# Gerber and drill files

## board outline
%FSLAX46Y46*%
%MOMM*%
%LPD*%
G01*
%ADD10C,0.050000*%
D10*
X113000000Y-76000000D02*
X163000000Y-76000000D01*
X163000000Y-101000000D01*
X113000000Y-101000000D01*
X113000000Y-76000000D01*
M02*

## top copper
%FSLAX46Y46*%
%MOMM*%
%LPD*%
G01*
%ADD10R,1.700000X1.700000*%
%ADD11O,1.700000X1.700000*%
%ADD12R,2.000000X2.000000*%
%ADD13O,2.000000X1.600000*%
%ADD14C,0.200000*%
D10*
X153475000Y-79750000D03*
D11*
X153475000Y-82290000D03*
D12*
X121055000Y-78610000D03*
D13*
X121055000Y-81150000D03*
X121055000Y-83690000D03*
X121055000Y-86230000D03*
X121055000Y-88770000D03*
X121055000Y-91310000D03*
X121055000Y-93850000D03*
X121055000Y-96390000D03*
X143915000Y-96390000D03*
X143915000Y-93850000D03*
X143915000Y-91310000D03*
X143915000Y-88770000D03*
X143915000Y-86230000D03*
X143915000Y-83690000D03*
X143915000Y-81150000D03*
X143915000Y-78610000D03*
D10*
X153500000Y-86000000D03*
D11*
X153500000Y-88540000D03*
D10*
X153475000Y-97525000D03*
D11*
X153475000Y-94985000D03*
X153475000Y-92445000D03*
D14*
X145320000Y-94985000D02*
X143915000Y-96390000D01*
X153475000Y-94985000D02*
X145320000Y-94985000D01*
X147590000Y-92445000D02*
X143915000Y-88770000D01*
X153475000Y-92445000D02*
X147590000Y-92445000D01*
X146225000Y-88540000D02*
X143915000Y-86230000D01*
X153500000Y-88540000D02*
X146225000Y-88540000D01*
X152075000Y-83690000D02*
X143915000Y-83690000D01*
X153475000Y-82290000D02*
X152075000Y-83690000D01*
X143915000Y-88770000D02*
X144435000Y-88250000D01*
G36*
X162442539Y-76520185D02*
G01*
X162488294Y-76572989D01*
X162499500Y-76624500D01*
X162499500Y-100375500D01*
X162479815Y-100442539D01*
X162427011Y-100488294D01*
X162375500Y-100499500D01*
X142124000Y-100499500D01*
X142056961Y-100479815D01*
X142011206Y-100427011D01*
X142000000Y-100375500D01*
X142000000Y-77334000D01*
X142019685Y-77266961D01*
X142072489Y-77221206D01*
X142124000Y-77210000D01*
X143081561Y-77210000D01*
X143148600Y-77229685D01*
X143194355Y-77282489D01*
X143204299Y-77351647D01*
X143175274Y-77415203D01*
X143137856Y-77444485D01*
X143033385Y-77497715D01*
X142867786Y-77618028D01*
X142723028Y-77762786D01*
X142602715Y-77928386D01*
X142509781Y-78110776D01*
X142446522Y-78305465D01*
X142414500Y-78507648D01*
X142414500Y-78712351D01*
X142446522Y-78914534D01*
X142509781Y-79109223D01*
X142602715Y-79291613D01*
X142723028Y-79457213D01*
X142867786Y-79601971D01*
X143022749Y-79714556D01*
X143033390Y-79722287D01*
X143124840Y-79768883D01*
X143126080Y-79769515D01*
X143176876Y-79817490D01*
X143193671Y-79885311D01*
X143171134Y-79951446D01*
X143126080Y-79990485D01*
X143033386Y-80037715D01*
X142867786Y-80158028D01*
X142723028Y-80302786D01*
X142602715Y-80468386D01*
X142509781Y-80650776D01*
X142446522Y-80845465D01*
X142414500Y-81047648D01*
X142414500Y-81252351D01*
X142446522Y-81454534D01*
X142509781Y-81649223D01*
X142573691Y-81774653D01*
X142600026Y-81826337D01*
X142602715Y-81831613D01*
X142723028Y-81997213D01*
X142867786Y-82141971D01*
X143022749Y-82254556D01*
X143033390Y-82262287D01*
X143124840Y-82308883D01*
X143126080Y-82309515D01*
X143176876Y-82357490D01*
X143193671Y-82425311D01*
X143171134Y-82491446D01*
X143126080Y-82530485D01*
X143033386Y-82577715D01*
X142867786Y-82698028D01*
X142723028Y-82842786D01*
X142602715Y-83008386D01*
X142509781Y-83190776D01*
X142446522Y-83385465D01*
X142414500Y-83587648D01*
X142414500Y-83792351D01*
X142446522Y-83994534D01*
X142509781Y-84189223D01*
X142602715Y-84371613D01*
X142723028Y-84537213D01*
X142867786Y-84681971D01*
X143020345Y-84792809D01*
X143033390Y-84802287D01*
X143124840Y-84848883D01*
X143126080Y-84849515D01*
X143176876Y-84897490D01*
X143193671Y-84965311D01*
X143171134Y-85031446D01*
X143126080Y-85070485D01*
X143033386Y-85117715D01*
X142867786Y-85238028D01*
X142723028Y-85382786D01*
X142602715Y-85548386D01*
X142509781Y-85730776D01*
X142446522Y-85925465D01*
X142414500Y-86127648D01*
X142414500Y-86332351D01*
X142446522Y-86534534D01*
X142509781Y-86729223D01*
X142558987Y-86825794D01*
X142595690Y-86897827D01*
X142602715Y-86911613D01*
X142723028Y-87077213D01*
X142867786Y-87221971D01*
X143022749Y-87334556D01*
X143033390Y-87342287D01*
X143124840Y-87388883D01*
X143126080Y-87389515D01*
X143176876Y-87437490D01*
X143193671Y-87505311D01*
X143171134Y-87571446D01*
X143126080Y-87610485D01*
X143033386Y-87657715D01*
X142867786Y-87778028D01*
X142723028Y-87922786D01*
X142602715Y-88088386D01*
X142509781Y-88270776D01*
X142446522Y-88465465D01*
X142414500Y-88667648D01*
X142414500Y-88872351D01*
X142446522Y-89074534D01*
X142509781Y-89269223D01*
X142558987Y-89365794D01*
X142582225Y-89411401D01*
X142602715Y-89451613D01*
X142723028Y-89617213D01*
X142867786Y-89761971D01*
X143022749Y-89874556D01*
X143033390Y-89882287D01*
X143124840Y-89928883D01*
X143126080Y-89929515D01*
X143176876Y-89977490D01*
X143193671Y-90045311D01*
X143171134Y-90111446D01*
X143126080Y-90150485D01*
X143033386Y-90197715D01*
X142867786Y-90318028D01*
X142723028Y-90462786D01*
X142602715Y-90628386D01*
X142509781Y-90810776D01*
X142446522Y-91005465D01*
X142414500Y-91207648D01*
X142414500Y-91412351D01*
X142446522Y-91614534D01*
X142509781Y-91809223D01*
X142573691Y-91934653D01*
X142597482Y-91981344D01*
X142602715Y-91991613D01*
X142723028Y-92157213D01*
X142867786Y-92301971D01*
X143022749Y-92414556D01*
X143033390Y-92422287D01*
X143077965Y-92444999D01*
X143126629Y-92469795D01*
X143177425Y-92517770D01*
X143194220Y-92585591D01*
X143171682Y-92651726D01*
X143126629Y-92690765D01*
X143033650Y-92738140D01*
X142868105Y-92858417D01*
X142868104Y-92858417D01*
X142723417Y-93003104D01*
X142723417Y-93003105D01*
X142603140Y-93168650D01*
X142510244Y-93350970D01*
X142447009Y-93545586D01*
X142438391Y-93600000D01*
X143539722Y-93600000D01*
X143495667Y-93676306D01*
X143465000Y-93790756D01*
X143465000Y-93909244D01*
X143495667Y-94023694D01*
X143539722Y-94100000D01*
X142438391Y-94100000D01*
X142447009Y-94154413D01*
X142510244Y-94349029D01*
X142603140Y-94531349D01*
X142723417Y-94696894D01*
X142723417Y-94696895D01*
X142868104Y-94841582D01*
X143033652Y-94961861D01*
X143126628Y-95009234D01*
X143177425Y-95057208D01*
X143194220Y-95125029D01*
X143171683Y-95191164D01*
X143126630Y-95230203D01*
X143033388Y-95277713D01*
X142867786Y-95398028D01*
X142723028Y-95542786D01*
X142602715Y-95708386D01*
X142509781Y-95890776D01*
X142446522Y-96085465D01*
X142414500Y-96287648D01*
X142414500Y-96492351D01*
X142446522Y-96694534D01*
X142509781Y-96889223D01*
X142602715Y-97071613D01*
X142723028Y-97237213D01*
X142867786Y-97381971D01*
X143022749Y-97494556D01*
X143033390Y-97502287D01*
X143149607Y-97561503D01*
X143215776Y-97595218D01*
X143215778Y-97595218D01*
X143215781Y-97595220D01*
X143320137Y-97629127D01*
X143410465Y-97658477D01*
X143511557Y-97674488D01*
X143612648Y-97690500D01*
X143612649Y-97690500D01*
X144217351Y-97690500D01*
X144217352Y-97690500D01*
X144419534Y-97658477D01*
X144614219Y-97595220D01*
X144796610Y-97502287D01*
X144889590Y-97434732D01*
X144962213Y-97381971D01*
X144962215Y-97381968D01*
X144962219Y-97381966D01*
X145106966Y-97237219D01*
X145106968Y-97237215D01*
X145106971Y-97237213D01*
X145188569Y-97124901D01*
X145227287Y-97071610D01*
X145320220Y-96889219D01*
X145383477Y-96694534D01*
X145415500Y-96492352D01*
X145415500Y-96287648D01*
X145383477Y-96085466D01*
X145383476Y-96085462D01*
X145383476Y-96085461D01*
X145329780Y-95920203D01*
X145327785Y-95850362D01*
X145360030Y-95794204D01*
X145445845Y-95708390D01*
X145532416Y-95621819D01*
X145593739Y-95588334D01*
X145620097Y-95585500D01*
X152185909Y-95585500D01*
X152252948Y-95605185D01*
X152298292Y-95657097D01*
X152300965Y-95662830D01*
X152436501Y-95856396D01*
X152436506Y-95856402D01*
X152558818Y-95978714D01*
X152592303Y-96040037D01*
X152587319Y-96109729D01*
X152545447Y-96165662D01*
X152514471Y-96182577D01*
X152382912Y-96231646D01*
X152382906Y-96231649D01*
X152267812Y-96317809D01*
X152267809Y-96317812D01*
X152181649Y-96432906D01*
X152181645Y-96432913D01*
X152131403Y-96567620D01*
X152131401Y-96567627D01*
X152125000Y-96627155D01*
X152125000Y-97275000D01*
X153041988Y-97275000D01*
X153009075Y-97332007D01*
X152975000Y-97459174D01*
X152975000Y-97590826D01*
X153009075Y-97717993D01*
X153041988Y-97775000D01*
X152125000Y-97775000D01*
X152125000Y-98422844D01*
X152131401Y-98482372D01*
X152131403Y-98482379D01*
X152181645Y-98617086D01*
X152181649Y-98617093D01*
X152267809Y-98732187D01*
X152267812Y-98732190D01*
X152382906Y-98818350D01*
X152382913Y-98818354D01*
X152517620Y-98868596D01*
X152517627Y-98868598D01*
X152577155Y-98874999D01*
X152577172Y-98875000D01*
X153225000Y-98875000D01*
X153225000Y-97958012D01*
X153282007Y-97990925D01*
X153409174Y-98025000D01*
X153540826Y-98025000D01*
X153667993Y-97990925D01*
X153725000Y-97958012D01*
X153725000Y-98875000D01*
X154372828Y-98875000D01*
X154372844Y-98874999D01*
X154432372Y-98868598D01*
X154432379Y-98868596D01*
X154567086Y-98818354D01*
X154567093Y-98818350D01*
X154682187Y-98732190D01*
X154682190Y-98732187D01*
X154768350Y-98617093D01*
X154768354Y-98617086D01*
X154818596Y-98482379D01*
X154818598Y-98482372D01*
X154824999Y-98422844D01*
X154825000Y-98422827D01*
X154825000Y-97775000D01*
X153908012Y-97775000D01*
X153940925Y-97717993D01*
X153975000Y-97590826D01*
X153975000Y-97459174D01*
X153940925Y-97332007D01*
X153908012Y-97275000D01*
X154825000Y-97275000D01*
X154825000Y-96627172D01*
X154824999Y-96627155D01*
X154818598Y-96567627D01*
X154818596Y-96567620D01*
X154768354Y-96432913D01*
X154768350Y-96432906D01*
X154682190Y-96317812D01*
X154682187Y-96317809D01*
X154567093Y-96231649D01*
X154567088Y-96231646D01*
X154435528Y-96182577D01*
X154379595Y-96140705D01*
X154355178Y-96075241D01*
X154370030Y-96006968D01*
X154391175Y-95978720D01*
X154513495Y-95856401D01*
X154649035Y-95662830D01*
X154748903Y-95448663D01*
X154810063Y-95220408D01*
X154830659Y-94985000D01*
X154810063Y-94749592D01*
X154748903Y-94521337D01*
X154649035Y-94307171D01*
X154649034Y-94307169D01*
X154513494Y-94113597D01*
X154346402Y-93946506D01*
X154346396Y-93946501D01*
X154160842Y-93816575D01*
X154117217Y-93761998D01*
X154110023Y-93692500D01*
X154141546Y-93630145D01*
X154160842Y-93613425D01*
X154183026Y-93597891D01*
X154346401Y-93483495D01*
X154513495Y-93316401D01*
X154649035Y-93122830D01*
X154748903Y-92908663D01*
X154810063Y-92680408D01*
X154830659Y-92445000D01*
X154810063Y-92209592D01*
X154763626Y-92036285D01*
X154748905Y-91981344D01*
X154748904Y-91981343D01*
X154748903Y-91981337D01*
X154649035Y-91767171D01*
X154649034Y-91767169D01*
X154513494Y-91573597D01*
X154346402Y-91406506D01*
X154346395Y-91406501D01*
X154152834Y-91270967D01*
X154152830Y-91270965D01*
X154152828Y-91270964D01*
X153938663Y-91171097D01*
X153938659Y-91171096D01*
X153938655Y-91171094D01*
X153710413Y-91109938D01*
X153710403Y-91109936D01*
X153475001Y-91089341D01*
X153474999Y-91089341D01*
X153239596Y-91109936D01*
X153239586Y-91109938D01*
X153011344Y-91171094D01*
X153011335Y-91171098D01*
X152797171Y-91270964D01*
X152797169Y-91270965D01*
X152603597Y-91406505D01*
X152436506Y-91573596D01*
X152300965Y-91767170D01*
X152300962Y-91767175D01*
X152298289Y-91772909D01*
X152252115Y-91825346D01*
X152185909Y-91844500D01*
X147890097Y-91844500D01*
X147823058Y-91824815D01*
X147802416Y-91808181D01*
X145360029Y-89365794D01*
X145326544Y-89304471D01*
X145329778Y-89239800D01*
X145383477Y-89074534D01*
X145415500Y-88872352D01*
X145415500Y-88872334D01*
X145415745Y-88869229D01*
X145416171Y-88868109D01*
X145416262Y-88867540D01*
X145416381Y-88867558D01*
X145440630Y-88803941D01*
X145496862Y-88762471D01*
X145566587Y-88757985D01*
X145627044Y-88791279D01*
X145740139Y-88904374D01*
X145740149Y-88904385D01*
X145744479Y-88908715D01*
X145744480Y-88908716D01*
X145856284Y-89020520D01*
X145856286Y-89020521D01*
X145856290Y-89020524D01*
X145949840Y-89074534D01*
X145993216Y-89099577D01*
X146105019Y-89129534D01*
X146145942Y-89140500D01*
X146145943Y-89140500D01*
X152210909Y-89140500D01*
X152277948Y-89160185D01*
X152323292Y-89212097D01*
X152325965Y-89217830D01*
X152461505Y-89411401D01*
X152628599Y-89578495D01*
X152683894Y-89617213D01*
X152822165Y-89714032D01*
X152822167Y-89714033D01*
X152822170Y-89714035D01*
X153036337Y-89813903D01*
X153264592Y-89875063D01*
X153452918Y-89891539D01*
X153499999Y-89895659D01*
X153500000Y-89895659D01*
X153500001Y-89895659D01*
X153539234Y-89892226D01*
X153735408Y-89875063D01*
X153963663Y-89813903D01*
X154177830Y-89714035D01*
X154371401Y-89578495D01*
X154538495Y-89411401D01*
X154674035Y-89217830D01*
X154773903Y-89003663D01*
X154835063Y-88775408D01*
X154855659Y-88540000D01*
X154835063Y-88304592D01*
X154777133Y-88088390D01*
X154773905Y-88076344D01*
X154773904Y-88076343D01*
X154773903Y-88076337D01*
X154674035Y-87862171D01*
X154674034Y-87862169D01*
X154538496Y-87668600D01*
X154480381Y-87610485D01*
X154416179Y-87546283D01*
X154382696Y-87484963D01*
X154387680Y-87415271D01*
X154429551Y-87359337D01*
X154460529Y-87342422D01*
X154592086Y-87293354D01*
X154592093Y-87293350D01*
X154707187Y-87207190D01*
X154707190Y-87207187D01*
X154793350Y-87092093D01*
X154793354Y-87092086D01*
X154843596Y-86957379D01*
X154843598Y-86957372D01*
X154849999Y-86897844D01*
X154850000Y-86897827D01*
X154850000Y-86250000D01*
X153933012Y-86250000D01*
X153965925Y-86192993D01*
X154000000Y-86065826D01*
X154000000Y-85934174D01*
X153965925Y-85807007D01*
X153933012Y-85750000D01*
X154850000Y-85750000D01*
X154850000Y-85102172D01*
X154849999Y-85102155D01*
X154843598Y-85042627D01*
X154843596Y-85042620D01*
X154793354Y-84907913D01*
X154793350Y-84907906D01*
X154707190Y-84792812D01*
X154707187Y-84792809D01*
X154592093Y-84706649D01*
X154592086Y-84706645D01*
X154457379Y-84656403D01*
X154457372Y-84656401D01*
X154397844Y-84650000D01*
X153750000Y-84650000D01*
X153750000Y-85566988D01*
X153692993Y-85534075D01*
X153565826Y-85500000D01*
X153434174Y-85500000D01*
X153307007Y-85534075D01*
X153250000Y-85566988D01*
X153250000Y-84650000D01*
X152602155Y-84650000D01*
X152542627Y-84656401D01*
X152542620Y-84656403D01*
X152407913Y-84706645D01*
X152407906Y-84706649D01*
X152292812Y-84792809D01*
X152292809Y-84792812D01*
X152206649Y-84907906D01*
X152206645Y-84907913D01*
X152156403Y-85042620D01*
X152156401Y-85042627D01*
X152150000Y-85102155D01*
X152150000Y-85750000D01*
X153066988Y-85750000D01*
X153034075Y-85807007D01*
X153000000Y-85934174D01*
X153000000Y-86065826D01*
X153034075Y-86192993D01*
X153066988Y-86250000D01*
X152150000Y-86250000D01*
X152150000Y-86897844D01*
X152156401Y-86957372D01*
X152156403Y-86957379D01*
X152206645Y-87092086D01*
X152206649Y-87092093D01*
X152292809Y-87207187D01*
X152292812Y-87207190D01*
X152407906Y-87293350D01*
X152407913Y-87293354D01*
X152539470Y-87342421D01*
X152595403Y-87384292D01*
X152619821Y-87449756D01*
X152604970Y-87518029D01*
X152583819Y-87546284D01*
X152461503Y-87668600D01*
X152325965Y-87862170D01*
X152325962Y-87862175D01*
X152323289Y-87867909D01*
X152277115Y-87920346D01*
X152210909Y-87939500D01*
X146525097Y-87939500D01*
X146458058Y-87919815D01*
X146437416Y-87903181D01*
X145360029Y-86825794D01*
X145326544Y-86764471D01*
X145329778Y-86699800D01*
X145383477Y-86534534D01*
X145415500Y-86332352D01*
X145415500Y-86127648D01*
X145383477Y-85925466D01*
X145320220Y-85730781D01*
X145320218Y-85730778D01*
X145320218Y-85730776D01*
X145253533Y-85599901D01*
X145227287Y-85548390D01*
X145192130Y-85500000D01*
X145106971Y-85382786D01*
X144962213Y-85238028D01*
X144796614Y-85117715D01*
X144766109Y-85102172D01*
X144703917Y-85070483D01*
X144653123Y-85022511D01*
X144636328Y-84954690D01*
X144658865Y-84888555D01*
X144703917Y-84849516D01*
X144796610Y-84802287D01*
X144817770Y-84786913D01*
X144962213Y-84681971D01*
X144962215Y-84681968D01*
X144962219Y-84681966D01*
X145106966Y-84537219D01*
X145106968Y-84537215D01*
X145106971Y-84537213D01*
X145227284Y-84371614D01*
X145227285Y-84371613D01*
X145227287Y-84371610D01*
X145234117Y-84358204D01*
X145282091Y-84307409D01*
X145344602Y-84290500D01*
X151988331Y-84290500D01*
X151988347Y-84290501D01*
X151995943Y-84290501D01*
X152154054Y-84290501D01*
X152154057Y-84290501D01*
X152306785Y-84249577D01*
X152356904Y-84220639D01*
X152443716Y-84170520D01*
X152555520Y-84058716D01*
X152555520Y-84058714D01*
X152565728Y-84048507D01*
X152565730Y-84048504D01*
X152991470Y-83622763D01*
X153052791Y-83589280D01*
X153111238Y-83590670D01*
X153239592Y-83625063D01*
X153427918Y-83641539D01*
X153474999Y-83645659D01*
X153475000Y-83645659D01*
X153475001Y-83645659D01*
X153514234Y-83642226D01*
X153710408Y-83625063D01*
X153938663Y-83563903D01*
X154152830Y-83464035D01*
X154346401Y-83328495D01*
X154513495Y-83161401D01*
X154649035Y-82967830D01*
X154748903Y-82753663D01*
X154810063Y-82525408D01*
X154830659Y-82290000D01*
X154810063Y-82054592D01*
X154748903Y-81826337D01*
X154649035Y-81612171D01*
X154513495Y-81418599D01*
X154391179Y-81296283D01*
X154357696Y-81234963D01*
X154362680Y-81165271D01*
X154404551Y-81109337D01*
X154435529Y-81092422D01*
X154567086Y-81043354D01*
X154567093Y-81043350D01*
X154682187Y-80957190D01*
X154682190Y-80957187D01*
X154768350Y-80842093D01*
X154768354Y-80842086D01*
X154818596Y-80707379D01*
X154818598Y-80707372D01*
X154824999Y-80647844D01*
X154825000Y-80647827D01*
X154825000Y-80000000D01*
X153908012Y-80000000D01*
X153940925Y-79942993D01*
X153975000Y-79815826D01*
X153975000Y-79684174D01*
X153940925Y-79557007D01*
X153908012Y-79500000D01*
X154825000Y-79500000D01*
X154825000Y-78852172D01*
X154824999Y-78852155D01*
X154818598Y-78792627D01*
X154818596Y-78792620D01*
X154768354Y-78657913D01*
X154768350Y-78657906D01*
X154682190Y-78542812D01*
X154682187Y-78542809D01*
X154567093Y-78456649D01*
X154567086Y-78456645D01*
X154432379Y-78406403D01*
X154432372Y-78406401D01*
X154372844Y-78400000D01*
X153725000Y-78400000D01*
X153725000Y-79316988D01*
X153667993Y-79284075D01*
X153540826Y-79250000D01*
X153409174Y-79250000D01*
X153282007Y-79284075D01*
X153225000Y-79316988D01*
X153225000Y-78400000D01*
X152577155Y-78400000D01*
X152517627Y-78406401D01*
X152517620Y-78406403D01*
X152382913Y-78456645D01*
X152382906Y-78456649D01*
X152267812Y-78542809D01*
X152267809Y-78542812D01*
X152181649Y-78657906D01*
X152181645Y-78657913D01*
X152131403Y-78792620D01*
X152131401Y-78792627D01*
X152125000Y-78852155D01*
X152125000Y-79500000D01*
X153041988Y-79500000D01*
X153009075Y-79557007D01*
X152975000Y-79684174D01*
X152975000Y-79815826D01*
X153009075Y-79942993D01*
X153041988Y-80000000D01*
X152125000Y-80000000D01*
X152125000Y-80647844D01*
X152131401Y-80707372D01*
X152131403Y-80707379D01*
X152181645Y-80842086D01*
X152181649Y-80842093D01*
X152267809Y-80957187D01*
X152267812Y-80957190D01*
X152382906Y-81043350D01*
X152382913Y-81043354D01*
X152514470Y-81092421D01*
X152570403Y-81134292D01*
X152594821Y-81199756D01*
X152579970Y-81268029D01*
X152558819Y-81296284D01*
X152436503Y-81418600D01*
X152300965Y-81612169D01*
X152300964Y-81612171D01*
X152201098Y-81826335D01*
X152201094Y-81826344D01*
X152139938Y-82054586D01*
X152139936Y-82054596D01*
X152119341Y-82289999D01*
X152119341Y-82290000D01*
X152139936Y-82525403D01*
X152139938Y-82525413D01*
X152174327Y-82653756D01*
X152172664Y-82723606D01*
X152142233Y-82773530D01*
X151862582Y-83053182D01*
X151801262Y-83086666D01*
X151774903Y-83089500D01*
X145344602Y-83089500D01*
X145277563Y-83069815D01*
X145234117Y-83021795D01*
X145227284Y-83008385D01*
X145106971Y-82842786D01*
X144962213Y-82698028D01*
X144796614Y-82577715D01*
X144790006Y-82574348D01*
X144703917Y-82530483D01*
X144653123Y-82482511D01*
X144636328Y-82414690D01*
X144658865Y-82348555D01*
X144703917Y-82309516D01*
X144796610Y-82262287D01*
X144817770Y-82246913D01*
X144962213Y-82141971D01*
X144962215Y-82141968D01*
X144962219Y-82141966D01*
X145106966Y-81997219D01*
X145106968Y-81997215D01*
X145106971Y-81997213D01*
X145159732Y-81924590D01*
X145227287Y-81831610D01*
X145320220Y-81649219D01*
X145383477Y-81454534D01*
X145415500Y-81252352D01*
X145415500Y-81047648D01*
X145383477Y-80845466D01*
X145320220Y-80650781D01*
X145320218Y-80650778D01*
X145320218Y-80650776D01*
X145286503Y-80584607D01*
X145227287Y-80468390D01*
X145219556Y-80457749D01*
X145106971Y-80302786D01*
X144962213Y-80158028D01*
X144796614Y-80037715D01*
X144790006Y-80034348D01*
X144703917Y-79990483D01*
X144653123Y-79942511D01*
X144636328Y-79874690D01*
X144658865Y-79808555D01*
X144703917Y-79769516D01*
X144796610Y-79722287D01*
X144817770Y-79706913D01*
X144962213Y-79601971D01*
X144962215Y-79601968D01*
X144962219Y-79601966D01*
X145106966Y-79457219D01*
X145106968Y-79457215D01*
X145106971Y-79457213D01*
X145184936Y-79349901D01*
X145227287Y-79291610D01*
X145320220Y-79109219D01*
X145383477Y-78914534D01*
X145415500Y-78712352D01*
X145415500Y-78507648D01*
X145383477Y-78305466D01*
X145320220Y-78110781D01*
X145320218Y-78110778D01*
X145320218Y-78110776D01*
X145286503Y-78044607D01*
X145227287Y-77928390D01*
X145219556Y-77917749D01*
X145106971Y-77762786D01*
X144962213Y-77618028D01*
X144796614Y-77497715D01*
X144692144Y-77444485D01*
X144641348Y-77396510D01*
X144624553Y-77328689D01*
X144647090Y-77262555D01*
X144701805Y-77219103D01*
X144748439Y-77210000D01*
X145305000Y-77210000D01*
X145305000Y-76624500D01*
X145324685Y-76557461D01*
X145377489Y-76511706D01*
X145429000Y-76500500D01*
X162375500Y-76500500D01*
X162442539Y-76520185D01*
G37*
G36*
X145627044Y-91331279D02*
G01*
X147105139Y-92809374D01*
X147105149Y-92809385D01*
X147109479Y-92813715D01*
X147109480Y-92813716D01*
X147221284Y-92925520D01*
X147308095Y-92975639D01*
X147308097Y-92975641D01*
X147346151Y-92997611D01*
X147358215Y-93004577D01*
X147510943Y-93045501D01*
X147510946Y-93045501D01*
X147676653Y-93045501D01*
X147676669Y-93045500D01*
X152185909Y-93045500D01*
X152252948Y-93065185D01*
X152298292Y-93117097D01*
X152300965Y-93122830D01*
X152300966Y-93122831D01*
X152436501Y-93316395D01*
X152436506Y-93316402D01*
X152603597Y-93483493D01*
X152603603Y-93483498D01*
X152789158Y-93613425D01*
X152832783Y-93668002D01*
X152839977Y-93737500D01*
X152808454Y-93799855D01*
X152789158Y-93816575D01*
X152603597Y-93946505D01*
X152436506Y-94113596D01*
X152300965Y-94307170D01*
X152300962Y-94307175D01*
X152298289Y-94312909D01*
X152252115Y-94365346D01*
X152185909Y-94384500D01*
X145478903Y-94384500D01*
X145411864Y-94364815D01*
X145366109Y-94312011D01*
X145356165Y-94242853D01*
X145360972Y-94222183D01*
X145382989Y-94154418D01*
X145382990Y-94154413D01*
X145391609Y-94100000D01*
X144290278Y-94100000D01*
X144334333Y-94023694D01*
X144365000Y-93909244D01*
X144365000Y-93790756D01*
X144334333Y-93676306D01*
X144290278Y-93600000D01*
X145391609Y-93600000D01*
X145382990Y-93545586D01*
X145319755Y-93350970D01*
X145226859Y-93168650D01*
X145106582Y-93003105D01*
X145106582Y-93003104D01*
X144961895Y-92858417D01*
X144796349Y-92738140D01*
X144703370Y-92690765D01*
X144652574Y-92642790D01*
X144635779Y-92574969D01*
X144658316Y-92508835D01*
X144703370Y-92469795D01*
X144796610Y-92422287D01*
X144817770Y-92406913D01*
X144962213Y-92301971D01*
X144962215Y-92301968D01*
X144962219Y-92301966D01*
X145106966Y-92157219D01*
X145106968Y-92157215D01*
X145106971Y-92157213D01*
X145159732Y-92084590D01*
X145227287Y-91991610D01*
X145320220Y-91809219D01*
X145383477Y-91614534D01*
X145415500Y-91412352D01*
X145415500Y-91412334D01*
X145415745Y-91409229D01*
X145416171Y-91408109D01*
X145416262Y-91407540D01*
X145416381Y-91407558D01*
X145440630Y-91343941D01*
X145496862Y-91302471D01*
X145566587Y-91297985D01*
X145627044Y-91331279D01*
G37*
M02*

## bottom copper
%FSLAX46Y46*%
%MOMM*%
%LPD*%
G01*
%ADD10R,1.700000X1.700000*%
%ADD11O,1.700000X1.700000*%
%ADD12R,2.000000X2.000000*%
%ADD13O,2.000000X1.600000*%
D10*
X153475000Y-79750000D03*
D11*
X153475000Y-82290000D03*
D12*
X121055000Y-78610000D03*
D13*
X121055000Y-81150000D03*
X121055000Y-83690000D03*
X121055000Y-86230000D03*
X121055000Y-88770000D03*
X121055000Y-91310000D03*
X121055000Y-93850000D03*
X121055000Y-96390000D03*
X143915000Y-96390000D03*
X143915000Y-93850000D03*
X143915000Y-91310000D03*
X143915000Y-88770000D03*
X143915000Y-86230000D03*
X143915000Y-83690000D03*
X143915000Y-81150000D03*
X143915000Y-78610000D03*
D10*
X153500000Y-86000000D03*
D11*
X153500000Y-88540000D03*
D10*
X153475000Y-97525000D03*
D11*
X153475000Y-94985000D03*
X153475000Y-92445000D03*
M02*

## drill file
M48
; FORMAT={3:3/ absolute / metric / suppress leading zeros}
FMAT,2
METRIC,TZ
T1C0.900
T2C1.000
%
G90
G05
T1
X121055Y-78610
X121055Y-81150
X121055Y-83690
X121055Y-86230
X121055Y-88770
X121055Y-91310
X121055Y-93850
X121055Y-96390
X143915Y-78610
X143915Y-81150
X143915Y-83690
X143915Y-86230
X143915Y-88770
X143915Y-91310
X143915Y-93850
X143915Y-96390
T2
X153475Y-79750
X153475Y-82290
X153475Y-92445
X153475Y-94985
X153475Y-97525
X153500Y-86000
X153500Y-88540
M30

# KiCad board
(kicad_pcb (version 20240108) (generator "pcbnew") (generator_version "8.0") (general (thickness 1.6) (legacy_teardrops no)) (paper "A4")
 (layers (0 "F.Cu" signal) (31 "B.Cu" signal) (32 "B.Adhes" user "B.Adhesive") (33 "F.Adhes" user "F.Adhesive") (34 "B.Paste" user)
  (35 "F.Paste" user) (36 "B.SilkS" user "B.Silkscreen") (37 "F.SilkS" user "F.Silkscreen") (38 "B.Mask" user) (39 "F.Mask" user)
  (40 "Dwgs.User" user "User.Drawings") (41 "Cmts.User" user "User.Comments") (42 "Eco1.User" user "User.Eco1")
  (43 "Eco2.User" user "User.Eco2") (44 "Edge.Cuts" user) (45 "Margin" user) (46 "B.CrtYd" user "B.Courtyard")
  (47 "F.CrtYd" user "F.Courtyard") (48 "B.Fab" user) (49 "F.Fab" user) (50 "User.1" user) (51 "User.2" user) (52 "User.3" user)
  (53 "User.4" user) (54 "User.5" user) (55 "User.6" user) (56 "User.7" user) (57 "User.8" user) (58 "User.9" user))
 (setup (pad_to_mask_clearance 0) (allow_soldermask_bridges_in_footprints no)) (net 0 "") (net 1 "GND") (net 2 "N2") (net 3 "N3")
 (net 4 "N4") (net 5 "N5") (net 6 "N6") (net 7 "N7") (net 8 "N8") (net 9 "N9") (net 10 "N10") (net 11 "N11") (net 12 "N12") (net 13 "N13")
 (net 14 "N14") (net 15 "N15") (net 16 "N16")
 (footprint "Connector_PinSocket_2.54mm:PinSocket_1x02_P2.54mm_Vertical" (layer "F.Cu") (at 153.475 79.75)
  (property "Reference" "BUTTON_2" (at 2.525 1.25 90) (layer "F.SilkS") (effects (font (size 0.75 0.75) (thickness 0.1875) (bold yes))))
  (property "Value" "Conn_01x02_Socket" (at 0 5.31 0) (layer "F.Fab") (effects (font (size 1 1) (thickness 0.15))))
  (pad "1" thru_hole rect (at 0 0) (size 1.7 1.7) (drill 1) (layers "*.Cu" "*.Mask") (remove_unused_layers no) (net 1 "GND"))
  (pad "2" thru_hole oval (at 0 2.54) (size 1.7 1.7) (drill 1) (layers "*.Cu" "*.Mask") (remove_unused_layers no) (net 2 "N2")))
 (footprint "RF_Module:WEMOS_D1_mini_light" (layer "F.Cu") (at 121.055 78.61)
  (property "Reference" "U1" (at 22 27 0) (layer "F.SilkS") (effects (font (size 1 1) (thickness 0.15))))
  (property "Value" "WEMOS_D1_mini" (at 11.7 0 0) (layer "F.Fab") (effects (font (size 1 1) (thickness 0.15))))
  (pad "1" thru_hole rect (at 0 0) (size 2 2) (drill 0.9) (layers "*.Cu" "*.Mask") (remove_unused_layers no) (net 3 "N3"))
  (pad "2" thru_hole oval (at 0 2.54) (size 2 1.6) (drill 0.9) (layers "*.Cu" "*.Mask") (remove_unused_layers no) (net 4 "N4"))
  (pad "3" thru_hole oval (at 0 5.08) (size 2 1.6) (drill 0.9) (layers "*.Cu" "*.Mask") (remove_unused_layers no) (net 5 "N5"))
  (pad "4" thru_hole oval (at 0 7.62) (size 2 1.6) (drill 0.9) (layers "*.Cu" "*.Mask") (remove_unused_layers no) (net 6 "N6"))
  (pad "5" thru_hole oval (at 0 10.16) (size 2 1.6) (drill 0.9) (layers "*.Cu" "*.Mask") (remove_unused_layers no) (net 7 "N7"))
  (pad "6" thru_hole oval (at 0 12.7) (size 2 1.6) (drill 0.9) (layers "*.Cu" "*.Mask") (remove_unused_layers no) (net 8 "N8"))
  (pad "7" thru_hole oval (at 0 15.24) (size 2 1.6) (drill 0.9) (layers "*.Cu" "*.Mask") (remove_unused_layers no) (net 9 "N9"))
  (pad "8" thru_hole oval (at 0 17.78) (size 2 1.6) (drill 0.9) (layers "*.Cu" "*.Mask") (remove_unused_layers no) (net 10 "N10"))
  (pad "9" thru_hole oval (at 22.86 17.78) (size 2 1.6) (drill 0.9) (layers "*.Cu" "*.Mask") (remove_unused_layers no) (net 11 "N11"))
  (pad "10" thru_hole oval (at 22.86 15.24) (size 2 1.6) (drill 0.9) (layers "*.Cu" "*.Mask") (remove_unused_layers no) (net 1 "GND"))
  (pad "11" thru_hole oval (at 22.86 12.7) (size 2 1.6) (drill 0.9) (layers "*.Cu" "*.Mask") (remove_unused_layers no) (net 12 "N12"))
  (pad "12" thru_hole oval (at 22.86 10.16) (size 2 1.6) (drill 0.9) (layers "*.Cu" "*.Mask") (remove_unused_layers no) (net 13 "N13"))
  (pad "13" thru_hole oval (at 22.86 7.62) (size 2 1.6) (drill 0.9) (layers "*.Cu" "*.Mask") (remove_unused_layers no) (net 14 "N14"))
  (pad "14" thru_hole oval (at 22.86 5.08) (size 2 1.6) (drill 0.9) (layers "*.Cu" "*.Mask") (remove_unused_layers no) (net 2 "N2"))
  (pad "15" thru_hole oval (at 22.86 2.54) (size 2 1.6) (drill 0.9) (layers "*.Cu" "*.Mask") (remove_unused_layers no) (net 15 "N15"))
  (pad "16" thru_hole oval (at 22.86 0) (size 2 1.6) (drill 0.9) (layers "*.Cu" "*.Mask") (remove_unused_layers no) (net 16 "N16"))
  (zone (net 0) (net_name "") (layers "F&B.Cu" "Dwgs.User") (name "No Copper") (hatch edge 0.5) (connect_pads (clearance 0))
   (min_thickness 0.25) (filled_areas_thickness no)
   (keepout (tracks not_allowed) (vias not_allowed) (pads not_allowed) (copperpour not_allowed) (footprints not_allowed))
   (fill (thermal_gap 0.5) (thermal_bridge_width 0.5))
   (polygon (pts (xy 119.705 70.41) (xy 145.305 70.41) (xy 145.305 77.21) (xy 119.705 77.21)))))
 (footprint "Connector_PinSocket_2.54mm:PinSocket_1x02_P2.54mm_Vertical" (layer "F.Cu") (at 153.5 86)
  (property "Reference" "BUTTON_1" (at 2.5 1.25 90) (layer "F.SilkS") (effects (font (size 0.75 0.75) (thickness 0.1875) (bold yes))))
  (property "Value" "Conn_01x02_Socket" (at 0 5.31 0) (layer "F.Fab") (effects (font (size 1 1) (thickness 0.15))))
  (pad "1" thru_hole rect (at 0 0) (size 1.7 1.7) (drill 1) (layers "*.Cu" "*.Mask") (remove_unused_layers no) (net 1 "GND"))
  (pad "2" thru_hole oval (at 0 2.54) (size 1.7 1.7) (drill 1) (layers "*.Cu" "*.Mask") (remove_unused_layers no) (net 14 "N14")))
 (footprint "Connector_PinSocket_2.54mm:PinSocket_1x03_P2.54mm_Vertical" (layer "F.Cu") (at 153.475 97.525 180)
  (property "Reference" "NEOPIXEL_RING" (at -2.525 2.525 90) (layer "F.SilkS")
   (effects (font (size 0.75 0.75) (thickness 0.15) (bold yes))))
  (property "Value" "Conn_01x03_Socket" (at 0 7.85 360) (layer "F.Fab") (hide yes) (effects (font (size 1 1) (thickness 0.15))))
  (pad "1" thru_hole rect (at 0 0 180) (size 1.7 1.7) (drill 1) (layers "*.Cu" "*.Mask") (remove_unused_layers no) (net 1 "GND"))
  (pad "2" thru_hole oval (at 0 2.54 180) (size 1.7 1.7) (drill 1) (layers "*.Cu" "*.Mask") (remove_unused_layers no) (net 11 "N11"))
  (pad "3" thru_hole oval (at 0 5.08 180) (size 1.7 1.7) (drill 1) (layers "*.Cu" "*.Mask") (remove_unused_layers no) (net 13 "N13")))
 (gr_rect (start 113 76) (end 163 101) (stroke (width 0.05) (type default)) (fill none) (layer "Edge.Cuts"))
 (segment (start 153.475 94.985) (end 145.32 94.985) (width 0.2) (layer "F.Cu") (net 11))
 (segment (start 145.32 94.985) (end 143.915 96.39) (width 0.2) (layer "F.Cu") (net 11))
 (segment (start 147.59 92.445) (end 143.915 88.77) (width 0.2) (layer "F.Cu") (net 13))
 (segment (start 143.915 88.77) (end 144.435 88.25) (width 0.2) (layer "F.Cu") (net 13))
 (segment (start 153.475 92.445) (end 147.59 92.445) (width 0.2) (layer "F.Cu") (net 13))
 (segment (start 152.075 83.69) (end 143.915 83.69) (width 0.2) (layer "F.Cu") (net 2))
 (segment (start 153.475 82.29) (end 152.075 83.69) (width 0.2) (layer "F.Cu") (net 2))
 (segment (start 153.5 88.54) (end 146.225 88.54) (width 0.2) (layer "F.Cu") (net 14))
 (segment (start 146.225 88.54) (end 143.915 86.23) (width 0.2) (layer "F.Cu") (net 14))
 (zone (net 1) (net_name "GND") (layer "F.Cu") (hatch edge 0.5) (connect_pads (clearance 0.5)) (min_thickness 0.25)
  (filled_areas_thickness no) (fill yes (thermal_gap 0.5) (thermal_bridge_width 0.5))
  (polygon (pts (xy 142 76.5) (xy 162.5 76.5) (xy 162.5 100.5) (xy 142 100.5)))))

